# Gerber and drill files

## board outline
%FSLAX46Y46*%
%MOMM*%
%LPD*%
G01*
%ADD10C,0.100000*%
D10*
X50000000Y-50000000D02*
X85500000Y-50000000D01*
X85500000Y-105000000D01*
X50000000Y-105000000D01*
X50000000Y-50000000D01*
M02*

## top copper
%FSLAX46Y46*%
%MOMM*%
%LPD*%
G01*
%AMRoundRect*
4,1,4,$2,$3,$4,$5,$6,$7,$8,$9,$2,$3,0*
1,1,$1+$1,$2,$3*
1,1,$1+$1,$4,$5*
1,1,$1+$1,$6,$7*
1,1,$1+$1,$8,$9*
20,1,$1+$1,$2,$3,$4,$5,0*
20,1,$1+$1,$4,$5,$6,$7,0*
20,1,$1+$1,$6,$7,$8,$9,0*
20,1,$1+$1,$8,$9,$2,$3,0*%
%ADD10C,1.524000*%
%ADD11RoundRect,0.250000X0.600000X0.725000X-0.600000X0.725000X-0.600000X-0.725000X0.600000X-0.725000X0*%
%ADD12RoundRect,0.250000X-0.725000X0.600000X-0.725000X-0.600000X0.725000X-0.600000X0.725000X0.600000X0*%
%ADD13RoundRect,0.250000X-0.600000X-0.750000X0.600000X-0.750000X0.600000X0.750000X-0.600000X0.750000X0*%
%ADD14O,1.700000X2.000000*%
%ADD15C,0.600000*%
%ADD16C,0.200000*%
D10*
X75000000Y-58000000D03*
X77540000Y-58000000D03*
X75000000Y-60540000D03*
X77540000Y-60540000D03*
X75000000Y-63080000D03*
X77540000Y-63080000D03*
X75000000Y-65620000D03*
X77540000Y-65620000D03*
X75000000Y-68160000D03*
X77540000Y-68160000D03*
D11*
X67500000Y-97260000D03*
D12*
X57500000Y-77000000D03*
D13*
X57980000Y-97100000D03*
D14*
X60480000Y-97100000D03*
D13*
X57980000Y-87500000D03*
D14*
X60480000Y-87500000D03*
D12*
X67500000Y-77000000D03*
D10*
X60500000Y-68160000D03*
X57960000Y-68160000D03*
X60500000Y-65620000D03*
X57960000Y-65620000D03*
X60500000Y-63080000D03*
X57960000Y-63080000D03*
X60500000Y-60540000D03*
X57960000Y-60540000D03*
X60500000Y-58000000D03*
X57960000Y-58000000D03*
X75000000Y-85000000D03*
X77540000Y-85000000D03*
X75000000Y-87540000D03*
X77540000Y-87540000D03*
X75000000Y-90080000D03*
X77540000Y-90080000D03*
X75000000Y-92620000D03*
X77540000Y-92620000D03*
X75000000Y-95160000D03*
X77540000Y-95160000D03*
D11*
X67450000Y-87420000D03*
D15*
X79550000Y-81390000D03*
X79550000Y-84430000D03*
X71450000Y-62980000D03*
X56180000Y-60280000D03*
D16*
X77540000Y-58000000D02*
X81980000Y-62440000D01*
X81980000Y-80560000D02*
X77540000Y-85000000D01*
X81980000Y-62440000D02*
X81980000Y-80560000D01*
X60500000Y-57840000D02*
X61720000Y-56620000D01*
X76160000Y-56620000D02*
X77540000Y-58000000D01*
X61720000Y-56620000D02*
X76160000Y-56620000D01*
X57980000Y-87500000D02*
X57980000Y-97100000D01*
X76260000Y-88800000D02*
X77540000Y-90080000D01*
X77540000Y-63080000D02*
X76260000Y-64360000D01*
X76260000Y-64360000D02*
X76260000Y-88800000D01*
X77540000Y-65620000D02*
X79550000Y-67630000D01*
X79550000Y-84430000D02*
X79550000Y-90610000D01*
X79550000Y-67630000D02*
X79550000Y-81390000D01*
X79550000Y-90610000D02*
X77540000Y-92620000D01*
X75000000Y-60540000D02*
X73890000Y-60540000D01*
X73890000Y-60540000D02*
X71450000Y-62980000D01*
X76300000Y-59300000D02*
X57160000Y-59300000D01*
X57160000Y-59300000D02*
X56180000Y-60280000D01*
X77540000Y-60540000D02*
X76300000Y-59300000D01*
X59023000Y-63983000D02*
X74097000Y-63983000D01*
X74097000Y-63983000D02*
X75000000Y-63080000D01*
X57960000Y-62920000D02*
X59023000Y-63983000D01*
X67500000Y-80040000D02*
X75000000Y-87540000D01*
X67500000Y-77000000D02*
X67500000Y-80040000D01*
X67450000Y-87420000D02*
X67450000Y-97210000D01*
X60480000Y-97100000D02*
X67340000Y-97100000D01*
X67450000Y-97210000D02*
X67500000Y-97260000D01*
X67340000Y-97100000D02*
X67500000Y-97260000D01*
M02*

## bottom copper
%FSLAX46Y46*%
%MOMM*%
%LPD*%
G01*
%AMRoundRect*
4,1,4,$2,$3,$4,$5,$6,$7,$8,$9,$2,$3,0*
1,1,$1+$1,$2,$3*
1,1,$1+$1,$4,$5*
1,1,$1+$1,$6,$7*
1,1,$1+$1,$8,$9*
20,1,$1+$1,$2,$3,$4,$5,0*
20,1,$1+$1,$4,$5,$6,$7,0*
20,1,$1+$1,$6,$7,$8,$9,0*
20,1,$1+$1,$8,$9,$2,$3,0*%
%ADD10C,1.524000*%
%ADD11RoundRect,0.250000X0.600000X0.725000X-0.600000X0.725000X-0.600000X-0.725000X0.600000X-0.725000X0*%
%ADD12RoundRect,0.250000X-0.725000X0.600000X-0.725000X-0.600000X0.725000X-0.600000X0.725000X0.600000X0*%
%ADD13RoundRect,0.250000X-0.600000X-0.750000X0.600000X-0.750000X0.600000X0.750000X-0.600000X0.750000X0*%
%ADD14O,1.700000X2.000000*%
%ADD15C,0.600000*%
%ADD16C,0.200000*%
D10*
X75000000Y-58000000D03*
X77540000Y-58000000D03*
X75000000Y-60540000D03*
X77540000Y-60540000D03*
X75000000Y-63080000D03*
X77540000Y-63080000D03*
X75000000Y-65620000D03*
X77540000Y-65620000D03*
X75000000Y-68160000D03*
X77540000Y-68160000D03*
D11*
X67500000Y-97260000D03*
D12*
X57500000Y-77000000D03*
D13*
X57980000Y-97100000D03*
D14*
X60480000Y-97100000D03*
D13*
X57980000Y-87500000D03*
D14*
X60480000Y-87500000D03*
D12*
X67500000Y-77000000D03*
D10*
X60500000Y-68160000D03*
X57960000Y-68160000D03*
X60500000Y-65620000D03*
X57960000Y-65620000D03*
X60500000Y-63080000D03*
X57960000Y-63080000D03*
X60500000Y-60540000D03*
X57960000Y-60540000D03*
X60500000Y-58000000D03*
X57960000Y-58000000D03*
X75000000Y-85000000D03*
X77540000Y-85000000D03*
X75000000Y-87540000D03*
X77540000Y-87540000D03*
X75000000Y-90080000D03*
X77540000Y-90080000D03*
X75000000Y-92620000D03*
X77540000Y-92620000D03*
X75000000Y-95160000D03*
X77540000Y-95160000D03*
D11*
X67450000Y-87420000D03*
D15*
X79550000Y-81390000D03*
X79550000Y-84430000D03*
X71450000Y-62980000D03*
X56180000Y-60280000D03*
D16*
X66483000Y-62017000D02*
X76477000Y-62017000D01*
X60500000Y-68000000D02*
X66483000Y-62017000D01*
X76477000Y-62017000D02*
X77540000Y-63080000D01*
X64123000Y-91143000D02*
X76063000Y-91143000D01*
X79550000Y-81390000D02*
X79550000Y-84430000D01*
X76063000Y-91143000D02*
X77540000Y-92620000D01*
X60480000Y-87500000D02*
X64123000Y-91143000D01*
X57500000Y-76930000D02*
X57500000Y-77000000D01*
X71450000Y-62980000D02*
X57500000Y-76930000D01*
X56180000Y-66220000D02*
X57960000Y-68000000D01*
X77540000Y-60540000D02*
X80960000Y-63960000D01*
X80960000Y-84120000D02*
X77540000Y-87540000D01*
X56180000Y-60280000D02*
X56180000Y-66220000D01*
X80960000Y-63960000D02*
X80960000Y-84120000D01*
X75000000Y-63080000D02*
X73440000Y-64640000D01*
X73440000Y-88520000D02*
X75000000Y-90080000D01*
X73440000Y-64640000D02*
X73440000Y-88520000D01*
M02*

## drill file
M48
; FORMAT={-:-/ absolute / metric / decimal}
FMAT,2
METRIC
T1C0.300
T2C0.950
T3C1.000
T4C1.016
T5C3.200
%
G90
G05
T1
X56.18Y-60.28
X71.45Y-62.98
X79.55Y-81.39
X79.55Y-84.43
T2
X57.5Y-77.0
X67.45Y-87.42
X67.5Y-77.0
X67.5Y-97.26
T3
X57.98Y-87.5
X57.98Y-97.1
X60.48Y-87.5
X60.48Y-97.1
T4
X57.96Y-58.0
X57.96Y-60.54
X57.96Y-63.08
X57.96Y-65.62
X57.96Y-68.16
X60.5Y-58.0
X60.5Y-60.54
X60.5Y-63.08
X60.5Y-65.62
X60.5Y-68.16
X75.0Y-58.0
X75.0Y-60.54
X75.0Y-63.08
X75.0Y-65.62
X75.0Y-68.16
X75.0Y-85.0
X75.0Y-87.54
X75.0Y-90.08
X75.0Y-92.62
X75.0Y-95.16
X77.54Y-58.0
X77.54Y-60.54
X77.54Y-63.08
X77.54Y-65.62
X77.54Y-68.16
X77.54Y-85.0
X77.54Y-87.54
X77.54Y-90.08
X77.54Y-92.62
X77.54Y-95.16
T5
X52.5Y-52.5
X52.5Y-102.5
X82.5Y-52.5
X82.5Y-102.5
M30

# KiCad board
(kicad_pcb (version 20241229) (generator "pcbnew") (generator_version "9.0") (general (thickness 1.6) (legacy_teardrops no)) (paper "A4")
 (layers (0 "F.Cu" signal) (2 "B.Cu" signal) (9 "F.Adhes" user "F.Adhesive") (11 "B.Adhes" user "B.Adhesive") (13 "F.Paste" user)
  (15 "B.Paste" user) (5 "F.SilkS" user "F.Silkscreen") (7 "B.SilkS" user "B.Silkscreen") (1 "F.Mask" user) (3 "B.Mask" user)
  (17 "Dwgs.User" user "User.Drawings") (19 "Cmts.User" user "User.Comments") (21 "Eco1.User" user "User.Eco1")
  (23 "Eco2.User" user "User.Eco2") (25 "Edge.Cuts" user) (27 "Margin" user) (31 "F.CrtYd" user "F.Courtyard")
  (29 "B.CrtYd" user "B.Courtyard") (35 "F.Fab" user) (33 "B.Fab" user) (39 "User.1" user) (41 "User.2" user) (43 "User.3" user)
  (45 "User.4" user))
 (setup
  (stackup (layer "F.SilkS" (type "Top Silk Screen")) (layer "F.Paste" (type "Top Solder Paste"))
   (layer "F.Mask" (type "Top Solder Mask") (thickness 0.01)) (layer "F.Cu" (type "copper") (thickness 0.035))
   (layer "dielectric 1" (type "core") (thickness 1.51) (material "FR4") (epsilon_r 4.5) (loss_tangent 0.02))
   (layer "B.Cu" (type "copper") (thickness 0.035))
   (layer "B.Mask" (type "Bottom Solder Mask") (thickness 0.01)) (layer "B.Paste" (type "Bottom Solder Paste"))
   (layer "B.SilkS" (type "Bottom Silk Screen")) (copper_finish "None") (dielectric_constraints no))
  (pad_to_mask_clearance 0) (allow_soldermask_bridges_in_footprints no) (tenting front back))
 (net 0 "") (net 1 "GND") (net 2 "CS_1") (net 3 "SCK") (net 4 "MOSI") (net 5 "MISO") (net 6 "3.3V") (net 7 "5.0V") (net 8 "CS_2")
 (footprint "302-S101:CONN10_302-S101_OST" (layer "F.Cu") (at 75 58 -90)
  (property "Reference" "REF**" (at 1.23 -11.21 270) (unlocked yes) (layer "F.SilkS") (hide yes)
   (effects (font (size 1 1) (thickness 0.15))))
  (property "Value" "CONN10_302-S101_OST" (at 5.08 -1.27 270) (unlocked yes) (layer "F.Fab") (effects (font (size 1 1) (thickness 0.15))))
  (pad "1" thru_hole circle (at 0 0 270) (size 1.524 1.524) (drill 1.016) (layers "*.Cu" "*.Mask") (remove_unused_layers no))
  (pad "2" thru_hole circle (at 0 -2.54 270) (size 1.524 1.524) (drill 1.016) (layers "*.Cu" "*.Mask") (remove_unused_layers no)
   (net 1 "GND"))
  (pad "3" thru_hole circle (at 2.54 0 270) (size 1.524 1.524) (drill 1.016) (layers "*.Cu" "*.Mask") (remove_unused_layers no)
   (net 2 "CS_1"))
  (pad "4" thru_hole circle (at 2.54 -2.54 270) (size 1.524 1.524) (drill 1.016) (layers "*.Cu" "*.Mask") (remove_unused_layers no)
   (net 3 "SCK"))
  (pad "5" thru_hole circle (at 5.08 0 270) (size 1.524 1.524) (drill 1.016) (layers "*.Cu" "*.Mask") (remove_unused_layers no)
   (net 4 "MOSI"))
  (pad "6" thru_hole circle (at 5.08 -2.54 270) (size 1.524 1.524) (drill 1.016) (layers "*.Cu" "*.Mask") (remove_unused_layers no)
   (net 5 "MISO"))
  (pad "7" thru_hole circle (at 7.62 0 270) (size 1.524 1.524) (drill 1.016) (layers "*.Cu" "*.Mask") (remove_unused_layers no))
  (pad "8" thru_hole circle (at 7.62 -2.54 270) (size 1.524 1.524) (drill 1.016) (layers "*.Cu" "*.Mask") (remove_unused_layers no)
   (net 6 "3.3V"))
  (pad "9" thru_hole circle (at 10.16 0 270) (size 1.524 1.524) (drill 1.016) (layers "*.Cu" "*.Mask") (remove_unused_layers no))
  (pad "10" thru_hole circle (at 10.16 -2.54 270) (size 1.524 1.524) (drill 1.016) (layers "*.Cu" "*.Mask") (remove_unused_layers no)))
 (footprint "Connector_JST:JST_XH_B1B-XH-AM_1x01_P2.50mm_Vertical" (layer "F.Cu") (at 67.5 97.26 180)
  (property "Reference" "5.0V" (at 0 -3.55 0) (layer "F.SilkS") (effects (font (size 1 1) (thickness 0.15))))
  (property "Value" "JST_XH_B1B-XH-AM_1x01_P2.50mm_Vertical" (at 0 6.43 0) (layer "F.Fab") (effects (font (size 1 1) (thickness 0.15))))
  (pad "1" thru_hole roundrect (at 0 0 180) (size 1.7 1.95) (drill 0.95) (layers "*.Cu" "*.Mask") (remove_unused_layers no)
   (roundrect_rratio 0.147059) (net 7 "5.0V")))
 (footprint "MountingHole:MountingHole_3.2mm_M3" (layer "F.Cu") (at 50.44 50.08)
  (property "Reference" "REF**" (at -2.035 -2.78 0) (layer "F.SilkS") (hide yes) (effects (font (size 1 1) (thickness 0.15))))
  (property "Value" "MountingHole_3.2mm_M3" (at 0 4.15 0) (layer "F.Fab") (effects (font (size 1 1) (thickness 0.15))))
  (pad "" np_thru_hole circle (at 2.06 2.42) (size 3.2 3.2) (drill 3.2) (layers "*.Cu" "*.Mask")))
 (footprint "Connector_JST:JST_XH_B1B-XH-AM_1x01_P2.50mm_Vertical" (layer "F.Cu") (at 57.5 77 -90)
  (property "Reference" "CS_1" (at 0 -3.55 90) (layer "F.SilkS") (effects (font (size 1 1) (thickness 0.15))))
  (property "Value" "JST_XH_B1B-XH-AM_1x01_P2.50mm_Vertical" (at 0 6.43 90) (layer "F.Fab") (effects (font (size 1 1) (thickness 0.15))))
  (pad "1" thru_hole roundrect (at 0 0 270) (size 1.7 1.95) (drill 0.95) (layers "*.Cu" "*.Mask") (remove_unused_layers no)
   (roundrect_rratio 0.147059) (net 2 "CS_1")))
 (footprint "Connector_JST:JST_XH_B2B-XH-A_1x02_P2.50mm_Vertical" (layer "F.Cu") (at 57.98 97.1)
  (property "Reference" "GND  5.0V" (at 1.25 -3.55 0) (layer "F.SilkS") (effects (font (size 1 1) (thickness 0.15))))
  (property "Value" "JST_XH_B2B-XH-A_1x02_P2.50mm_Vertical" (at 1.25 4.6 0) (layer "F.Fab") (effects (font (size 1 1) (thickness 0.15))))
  (pad "1" thru_hole roundrect (at 0 0) (size 1.7 2) (drill 1) (layers "*.Cu" "*.Mask") (remove_unused_layers no)
   (roundrect_rratio 0.147059) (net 1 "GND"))
  (pad "2" thru_hole oval (at 2.5 0) (size 1.7 2) (drill 1) (layers "*.Cu" "*.Mask") (remove_unused_layers no) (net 7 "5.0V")))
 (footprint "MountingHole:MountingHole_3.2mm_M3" (layer "F.Cu") (at 84.75 50.83)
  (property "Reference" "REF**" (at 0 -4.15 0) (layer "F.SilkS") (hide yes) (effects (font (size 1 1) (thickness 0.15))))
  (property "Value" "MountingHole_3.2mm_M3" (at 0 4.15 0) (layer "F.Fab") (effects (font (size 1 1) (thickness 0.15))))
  (pad "" np_thru_hole circle (at -2.25 1.67) (size 3.2 3.2) (drill 3.2) (layers "*.Cu" "*.Mask")))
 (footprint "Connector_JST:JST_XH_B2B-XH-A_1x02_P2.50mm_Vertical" (layer "F.Cu") (at 57.98 87.5)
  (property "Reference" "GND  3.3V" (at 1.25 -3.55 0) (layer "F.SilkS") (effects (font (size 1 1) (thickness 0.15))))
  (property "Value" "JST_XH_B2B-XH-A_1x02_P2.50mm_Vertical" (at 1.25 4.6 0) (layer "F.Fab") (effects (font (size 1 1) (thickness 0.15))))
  (pad "1" thru_hole roundrect (at 0 0) (size 1.7 2) (drill 1) (layers "*.Cu" "*.Mask") (remove_unused_layers no)
   (roundrect_rratio 0.147059) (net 1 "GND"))
  (pad "2" thru_hole oval (at 2.5 0) (size 1.7 2) (drill 1) (layers "*.Cu" "*.Mask") (remove_unused_layers no) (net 6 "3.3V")))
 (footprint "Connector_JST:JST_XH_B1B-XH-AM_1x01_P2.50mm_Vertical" (layer "F.Cu") (at 67.5 77 -90)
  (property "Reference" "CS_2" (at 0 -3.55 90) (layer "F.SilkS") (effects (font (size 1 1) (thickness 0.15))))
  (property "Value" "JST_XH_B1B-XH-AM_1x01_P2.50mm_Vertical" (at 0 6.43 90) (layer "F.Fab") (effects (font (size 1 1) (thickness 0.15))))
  (pad "1" thru_hole roundrect (at 0 0 270) (size 1.7 1.95) (drill 0.95) (layers "*.Cu" "*.Mask") (remove_unused_layers no)
   (roundrect_rratio 0.147059) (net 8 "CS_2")))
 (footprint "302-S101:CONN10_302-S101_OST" (layer "F.Cu") (at 60.5 68.16 90)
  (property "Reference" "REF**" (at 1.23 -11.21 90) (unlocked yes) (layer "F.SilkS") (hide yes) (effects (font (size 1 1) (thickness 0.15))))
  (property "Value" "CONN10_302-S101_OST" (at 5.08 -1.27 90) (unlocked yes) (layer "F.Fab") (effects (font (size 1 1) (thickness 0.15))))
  (pad "1" thru_hole circle (at 0 0 90) (size 1.524 1.524) (drill 1.016) (layers "*.Cu" "*.Mask") (remove_unused_layers no) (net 5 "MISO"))
  (pad "2" thru_hole circle (at 0 -2.54 90) (size 1.524 1.524) (drill 1.016) (layers "*.Cu" "*.Mask") (remove_unused_layers no)
   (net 3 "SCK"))
  (pad "3" thru_hole circle (at 2.54 0 90) (size 1.524 1.524) (drill 1.016) (layers "*.Cu" "*.Mask") (remove_unused_layers no))
  (pad "4" thru_hole circle (at 2.54 -2.54 90) (size 1.524 1.524) (drill 1.016) (layers "*.Cu" "*.Mask") (remove_unused_layers no))
  (pad "5" thru_hole circle (at 5.08 0 90) (size 1.524 1.524) (drill 1.016) (layers "*.Cu" "*.Mask") (remove_unused_layers no))
  (pad "6" thru_hole circle (at 5.08 -2.54 90) (size 1.524 1.524) (drill 1.016) (layers "*.Cu" "*.Mask") (remove_unused_layers no)
   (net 4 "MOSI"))
  (pad "7" thru_hole circle (at 7.62 0 90) (size 1.524 1.524) (drill 1.016) (layers "*.Cu" "*.Mask") (remove_unused_layers no))
  (pad "8" thru_hole circle (at 7.62 -2.54 90) (size 1.524 1.524) (drill 1.016) (layers "*.Cu" "*.Mask") (remove_unused_layers no))
  (pad "9" thru_hole circle (at 10.16 0 90) (size 1.524 1.524) (drill 1.016) (layers "*.Cu" "*.Mask") (remove_unused_layers no)
   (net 1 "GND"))
  (pad "10" thru_hole circle (at 10.16 -2.54 90) (size 1.524 1.524) (drill 1.016) (layers "*.Cu" "*.Mask") (remove_unused_layers no)))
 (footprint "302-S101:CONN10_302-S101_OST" (layer "F.Cu") (at 75 85 -90)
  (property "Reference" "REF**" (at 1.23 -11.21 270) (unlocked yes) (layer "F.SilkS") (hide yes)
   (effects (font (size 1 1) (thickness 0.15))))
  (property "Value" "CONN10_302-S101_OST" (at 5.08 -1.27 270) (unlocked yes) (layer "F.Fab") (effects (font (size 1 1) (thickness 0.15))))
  (pad "1" thru_hole circle (at 0 0 270) (size 1.524 1.524) (drill 1.016) (layers "*.Cu" "*.Mask") (remove_unused_layers no))
  (pad "2" thru_hole circle (at 0 -2.54 270) (size 1.524 1.524) (drill 1.016) (layers "*.Cu" "*.Mask") (remove_unused_layers no)
   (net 1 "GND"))
  (pad "3" thru_hole circle (at 2.54 0 270) (size 1.524 1.524) (drill 1.016) (layers "*.Cu" "*.Mask") (remove_unused_layers no)
   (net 8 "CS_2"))
  (pad "4" thru_hole circle (at 2.54 -2.54 270) (size 1.524 1.524) (drill 1.016) (layers "*.Cu" "*.Mask") (remove_unused_layers no)
   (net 3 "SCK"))
  (pad "5" thru_hole circle (at 5.08 0 270) (size 1.524 1.524) (drill 1.016) (layers "*.Cu" "*.Mask") (remove_unused_layers no)
   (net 4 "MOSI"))
  (pad "6" thru_hole circle (at 5.08 -2.54 270) (size 1.524 1.524) (drill 1.016) (layers "*.Cu" "*.Mask") (remove_unused_layers no)
   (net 5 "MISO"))
  (pad "7" thru_hole circle (at 7.62 0 270) (size 1.524 1.524) (drill 1.016) (layers "*.Cu" "*.Mask") (remove_unused_layers no))
  (pad "8" thru_hole circle (at 7.62 -2.54 270) (size 1.524 1.524) (drill 1.016) (layers "*.Cu" "*.Mask") (remove_unused_layers no)
   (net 6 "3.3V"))
  (pad "9" thru_hole circle (at 10.16 0 270) (size 1.524 1.524) (drill 1.016) (layers "*.Cu" "*.Mask") (remove_unused_layers no))
  (pad "10" thru_hole circle (at 10.16 -2.54 270) (size 1.524 1.524) (drill 1.016) (layers "*.Cu" "*.Mask") (remove_unused_layers no)))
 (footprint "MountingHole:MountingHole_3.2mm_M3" (layer "F.Cu") (at 172.12 53.48)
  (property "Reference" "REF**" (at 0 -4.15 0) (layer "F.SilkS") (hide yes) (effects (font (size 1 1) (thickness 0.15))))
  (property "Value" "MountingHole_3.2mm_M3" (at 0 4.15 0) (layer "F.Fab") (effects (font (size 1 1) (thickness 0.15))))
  (pad "" np_thru_hole circle (at -119.62 49.02) (size 3.2 3.2) (drill 3.2) (layers "*.Cu" "*.Mask")))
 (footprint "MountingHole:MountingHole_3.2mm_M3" (layer "F.Cu") (at 83.83 102.93)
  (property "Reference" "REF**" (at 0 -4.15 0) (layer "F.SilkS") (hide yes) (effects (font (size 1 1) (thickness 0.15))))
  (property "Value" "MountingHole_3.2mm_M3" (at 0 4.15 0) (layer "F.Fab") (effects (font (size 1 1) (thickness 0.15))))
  (pad "" np_thru_hole circle (at -1.33 -0.43) (size 3.2 3.2) (drill 3.2) (layers "*.Cu" "*.Mask")))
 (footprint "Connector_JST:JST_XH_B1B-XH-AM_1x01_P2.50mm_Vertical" (layer "F.Cu") (at 67.45 87.42 180)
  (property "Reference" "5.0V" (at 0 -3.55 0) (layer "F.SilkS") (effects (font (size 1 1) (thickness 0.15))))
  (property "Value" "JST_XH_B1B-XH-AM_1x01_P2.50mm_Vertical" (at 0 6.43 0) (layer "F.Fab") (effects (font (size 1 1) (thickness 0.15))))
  (pad "1" thru_hole roundrect (at 0 0 180) (size 1.7 1.95) (drill 0.95) (layers "*.Cu" "*.Mask") (remove_unused_layers no)
   (roundrect_rratio 0.147059) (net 7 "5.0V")))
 (gr_rect (start 50 50) (end 85.5 105) (stroke (width 0.1) (type solid)) (fill no) (layer "Edge.Cuts"))
 (segment (start 77.54 58) (end 81.98 62.44) (width 0.2) (layer "F.Cu") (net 1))
 (segment (start 81.98 80.56) (end 77.54 85) (width 0.2) (layer "F.Cu") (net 1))
 (segment (start 81.98 62.44) (end 81.98 80.56) (width 0.2) (layer "F.Cu") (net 1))
 (segment (start 60.5 57.84) (end 61.72 56.62) (width 0.2) (layer "F.Cu") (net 1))
 (segment (start 76.16 56.62) (end 77.54 58) (width 0.2) (layer "F.Cu") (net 1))
 (segment (start 61.72 56.62) (end 76.16 56.62) (width 0.2) (layer "F.Cu") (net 1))
 (segment (start 57.98 87.5) (end 57.98 97.1) (width 0.2) (layer "F.Cu") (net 1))
 (segment (start 76.26 88.8) (end 77.54 90.08) (width 0.2) (layer "F.Cu") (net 5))
 (segment (start 77.54 63.08) (end 76.26 64.36) (width 0.2) (layer "F.Cu") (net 5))
 (segment (start 76.26 64.36) (end 76.26 88.8) (width 0.2) (layer "F.Cu") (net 5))
 (segment (start 66.483 62.017) (end 76.477 62.017) (width 0.2) (layer "B.Cu") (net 5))
 (segment (start 60.5 68) (end 66.483 62.017) (width 0.2) (layer "B.Cu") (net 5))
 (segment (start 76.477 62.017) (end 77.54 63.08) (width 0.2) (layer "B.Cu") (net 5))
 (segment (start 77.54 65.62) (end 79.55 67.63) (width 0.2) (layer "F.Cu") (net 6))
 (segment (start 79.55 84.43) (end 79.55 90.61) (width 0.2) (layer "F.Cu") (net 6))
 (segment (start 79.55 67.63) (end 79.55 81.39) (width 0.2) (layer "F.Cu") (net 6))
 (segment (start 79.55 90.61) (end 77.54 92.62) (width 0.2) (layer "F.Cu") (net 6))
 (via (at 79.55 81.39) (size 0.6) (drill 0.3) (layers "F.Cu" "B.Cu") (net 6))
 (via (at 79.55 84.43) (size 0.6) (drill 0.3) (layers "F.Cu" "B.Cu") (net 6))
 (segment (start 64.123 91.143) (end 76.063 91.143) (width 0.2) (layer "B.Cu") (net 6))
 (segment (start 79.55 81.39) (end 79.55 84.43) (width 0.2) (layer "B.Cu") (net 6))
 (segment (start 76.063 91.143) (end 77.54 92.62) (width 0.2) (layer "B.Cu") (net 6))
 (segment (start 60.48 87.5) (end 64.123 91.143) (width 0.2) (layer "B.Cu") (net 6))
 (segment (start 75 60.54) (end 73.89 60.54) (width 0.2) (layer "F.Cu") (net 2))
 (segment (start 73.89 60.54) (end 71.45 62.98) (width 0.2) (layer "F.Cu") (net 2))
 (via (at 71.45 62.98) (size 0.6) (drill 0.3) (layers "F.Cu" "B.Cu") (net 2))
 (segment (start 57.5 76.93) (end 57.5 77) (width 0.2) (layer "B.Cu") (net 2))
 (segment (start 71.45 62.98) (end 57.5 76.93) (width 0.2) (layer "B.Cu") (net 2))
 (segment (start 76.3 59.3) (end 57.16 59.3) (width 0.2) (layer "F.Cu") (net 3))
 (segment (start 57.16 59.3) (end 56.18 60.28) (width 0.2) (layer "F.Cu") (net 3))
 (segment (start 77.54 60.54) (end 76.3 59.3) (width 0.2) (layer "F.Cu") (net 3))
 (via (at 56.18 60.28) (size 0.6) (drill 0.3) (layers "F.Cu" "B.Cu") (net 3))
 (segment (start 56.18 66.22) (end 57.96 68) (width 0.2) (layer "B.Cu") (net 3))
 (segment (start 77.54 60.54) (end 80.96 63.96) (width 0.2) (layer "B.Cu") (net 3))
 (segment (start 80.96 84.12) (end 77.54 87.54) (width 0.2) (layer "B.Cu") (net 3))
 (segment (start 56.18 60.28) (end 56.18 66.22) (width 0.2) (layer "B.Cu") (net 3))
 (segment (start 80.96 63.96) (end 80.96 84.12) (width 0.2) (layer "B.Cu") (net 3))
 (segment (start 59.023 63.983) (end 74.097 63.983) (width 0.2) (layer "F.Cu") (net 4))
 (segment (start 74.097 63.983) (end 75 63.08) (width 0.2) (layer "F.Cu") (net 4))
 (segment (start 57.96 62.92) (end 59.023 63.983) (width 0.2) (layer "F.Cu") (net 4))
 (segment (start 75 63.08) (end 73.44 64.64) (width 0.2) (layer "B.Cu") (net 4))
 (segment (start 73.44 88.52) (end 75 90.08) (width 0.2) (layer "B.Cu") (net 4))
 (segment (start 73.44 64.64) (end 73.44 88.52) (width 0.2) (layer "B.Cu") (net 4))
 (segment (start 67.5 80.04) (end 75 87.54) (width 0.2) (layer "F.Cu") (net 8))
 (segment (start 67.5 77) (end 67.5 80.04) (width 0.2) (layer "F.Cu") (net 8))
 (segment (start 67.45 87.42) (end 67.45 97.21) (width 0.2) (layer "F.Cu") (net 7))
 (segment (start 60.48 97.1) (end 67.34 97.1) (width 0.2) (layer "F.Cu") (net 7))
 (segment (start 67.45 97.21) (end 67.5 97.26) (width 0.2) (layer "F.Cu") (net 7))
 (segment (start 67.34 97.1) (end 67.5 97.26) (width 0.2) (layer "F.Cu") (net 7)))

